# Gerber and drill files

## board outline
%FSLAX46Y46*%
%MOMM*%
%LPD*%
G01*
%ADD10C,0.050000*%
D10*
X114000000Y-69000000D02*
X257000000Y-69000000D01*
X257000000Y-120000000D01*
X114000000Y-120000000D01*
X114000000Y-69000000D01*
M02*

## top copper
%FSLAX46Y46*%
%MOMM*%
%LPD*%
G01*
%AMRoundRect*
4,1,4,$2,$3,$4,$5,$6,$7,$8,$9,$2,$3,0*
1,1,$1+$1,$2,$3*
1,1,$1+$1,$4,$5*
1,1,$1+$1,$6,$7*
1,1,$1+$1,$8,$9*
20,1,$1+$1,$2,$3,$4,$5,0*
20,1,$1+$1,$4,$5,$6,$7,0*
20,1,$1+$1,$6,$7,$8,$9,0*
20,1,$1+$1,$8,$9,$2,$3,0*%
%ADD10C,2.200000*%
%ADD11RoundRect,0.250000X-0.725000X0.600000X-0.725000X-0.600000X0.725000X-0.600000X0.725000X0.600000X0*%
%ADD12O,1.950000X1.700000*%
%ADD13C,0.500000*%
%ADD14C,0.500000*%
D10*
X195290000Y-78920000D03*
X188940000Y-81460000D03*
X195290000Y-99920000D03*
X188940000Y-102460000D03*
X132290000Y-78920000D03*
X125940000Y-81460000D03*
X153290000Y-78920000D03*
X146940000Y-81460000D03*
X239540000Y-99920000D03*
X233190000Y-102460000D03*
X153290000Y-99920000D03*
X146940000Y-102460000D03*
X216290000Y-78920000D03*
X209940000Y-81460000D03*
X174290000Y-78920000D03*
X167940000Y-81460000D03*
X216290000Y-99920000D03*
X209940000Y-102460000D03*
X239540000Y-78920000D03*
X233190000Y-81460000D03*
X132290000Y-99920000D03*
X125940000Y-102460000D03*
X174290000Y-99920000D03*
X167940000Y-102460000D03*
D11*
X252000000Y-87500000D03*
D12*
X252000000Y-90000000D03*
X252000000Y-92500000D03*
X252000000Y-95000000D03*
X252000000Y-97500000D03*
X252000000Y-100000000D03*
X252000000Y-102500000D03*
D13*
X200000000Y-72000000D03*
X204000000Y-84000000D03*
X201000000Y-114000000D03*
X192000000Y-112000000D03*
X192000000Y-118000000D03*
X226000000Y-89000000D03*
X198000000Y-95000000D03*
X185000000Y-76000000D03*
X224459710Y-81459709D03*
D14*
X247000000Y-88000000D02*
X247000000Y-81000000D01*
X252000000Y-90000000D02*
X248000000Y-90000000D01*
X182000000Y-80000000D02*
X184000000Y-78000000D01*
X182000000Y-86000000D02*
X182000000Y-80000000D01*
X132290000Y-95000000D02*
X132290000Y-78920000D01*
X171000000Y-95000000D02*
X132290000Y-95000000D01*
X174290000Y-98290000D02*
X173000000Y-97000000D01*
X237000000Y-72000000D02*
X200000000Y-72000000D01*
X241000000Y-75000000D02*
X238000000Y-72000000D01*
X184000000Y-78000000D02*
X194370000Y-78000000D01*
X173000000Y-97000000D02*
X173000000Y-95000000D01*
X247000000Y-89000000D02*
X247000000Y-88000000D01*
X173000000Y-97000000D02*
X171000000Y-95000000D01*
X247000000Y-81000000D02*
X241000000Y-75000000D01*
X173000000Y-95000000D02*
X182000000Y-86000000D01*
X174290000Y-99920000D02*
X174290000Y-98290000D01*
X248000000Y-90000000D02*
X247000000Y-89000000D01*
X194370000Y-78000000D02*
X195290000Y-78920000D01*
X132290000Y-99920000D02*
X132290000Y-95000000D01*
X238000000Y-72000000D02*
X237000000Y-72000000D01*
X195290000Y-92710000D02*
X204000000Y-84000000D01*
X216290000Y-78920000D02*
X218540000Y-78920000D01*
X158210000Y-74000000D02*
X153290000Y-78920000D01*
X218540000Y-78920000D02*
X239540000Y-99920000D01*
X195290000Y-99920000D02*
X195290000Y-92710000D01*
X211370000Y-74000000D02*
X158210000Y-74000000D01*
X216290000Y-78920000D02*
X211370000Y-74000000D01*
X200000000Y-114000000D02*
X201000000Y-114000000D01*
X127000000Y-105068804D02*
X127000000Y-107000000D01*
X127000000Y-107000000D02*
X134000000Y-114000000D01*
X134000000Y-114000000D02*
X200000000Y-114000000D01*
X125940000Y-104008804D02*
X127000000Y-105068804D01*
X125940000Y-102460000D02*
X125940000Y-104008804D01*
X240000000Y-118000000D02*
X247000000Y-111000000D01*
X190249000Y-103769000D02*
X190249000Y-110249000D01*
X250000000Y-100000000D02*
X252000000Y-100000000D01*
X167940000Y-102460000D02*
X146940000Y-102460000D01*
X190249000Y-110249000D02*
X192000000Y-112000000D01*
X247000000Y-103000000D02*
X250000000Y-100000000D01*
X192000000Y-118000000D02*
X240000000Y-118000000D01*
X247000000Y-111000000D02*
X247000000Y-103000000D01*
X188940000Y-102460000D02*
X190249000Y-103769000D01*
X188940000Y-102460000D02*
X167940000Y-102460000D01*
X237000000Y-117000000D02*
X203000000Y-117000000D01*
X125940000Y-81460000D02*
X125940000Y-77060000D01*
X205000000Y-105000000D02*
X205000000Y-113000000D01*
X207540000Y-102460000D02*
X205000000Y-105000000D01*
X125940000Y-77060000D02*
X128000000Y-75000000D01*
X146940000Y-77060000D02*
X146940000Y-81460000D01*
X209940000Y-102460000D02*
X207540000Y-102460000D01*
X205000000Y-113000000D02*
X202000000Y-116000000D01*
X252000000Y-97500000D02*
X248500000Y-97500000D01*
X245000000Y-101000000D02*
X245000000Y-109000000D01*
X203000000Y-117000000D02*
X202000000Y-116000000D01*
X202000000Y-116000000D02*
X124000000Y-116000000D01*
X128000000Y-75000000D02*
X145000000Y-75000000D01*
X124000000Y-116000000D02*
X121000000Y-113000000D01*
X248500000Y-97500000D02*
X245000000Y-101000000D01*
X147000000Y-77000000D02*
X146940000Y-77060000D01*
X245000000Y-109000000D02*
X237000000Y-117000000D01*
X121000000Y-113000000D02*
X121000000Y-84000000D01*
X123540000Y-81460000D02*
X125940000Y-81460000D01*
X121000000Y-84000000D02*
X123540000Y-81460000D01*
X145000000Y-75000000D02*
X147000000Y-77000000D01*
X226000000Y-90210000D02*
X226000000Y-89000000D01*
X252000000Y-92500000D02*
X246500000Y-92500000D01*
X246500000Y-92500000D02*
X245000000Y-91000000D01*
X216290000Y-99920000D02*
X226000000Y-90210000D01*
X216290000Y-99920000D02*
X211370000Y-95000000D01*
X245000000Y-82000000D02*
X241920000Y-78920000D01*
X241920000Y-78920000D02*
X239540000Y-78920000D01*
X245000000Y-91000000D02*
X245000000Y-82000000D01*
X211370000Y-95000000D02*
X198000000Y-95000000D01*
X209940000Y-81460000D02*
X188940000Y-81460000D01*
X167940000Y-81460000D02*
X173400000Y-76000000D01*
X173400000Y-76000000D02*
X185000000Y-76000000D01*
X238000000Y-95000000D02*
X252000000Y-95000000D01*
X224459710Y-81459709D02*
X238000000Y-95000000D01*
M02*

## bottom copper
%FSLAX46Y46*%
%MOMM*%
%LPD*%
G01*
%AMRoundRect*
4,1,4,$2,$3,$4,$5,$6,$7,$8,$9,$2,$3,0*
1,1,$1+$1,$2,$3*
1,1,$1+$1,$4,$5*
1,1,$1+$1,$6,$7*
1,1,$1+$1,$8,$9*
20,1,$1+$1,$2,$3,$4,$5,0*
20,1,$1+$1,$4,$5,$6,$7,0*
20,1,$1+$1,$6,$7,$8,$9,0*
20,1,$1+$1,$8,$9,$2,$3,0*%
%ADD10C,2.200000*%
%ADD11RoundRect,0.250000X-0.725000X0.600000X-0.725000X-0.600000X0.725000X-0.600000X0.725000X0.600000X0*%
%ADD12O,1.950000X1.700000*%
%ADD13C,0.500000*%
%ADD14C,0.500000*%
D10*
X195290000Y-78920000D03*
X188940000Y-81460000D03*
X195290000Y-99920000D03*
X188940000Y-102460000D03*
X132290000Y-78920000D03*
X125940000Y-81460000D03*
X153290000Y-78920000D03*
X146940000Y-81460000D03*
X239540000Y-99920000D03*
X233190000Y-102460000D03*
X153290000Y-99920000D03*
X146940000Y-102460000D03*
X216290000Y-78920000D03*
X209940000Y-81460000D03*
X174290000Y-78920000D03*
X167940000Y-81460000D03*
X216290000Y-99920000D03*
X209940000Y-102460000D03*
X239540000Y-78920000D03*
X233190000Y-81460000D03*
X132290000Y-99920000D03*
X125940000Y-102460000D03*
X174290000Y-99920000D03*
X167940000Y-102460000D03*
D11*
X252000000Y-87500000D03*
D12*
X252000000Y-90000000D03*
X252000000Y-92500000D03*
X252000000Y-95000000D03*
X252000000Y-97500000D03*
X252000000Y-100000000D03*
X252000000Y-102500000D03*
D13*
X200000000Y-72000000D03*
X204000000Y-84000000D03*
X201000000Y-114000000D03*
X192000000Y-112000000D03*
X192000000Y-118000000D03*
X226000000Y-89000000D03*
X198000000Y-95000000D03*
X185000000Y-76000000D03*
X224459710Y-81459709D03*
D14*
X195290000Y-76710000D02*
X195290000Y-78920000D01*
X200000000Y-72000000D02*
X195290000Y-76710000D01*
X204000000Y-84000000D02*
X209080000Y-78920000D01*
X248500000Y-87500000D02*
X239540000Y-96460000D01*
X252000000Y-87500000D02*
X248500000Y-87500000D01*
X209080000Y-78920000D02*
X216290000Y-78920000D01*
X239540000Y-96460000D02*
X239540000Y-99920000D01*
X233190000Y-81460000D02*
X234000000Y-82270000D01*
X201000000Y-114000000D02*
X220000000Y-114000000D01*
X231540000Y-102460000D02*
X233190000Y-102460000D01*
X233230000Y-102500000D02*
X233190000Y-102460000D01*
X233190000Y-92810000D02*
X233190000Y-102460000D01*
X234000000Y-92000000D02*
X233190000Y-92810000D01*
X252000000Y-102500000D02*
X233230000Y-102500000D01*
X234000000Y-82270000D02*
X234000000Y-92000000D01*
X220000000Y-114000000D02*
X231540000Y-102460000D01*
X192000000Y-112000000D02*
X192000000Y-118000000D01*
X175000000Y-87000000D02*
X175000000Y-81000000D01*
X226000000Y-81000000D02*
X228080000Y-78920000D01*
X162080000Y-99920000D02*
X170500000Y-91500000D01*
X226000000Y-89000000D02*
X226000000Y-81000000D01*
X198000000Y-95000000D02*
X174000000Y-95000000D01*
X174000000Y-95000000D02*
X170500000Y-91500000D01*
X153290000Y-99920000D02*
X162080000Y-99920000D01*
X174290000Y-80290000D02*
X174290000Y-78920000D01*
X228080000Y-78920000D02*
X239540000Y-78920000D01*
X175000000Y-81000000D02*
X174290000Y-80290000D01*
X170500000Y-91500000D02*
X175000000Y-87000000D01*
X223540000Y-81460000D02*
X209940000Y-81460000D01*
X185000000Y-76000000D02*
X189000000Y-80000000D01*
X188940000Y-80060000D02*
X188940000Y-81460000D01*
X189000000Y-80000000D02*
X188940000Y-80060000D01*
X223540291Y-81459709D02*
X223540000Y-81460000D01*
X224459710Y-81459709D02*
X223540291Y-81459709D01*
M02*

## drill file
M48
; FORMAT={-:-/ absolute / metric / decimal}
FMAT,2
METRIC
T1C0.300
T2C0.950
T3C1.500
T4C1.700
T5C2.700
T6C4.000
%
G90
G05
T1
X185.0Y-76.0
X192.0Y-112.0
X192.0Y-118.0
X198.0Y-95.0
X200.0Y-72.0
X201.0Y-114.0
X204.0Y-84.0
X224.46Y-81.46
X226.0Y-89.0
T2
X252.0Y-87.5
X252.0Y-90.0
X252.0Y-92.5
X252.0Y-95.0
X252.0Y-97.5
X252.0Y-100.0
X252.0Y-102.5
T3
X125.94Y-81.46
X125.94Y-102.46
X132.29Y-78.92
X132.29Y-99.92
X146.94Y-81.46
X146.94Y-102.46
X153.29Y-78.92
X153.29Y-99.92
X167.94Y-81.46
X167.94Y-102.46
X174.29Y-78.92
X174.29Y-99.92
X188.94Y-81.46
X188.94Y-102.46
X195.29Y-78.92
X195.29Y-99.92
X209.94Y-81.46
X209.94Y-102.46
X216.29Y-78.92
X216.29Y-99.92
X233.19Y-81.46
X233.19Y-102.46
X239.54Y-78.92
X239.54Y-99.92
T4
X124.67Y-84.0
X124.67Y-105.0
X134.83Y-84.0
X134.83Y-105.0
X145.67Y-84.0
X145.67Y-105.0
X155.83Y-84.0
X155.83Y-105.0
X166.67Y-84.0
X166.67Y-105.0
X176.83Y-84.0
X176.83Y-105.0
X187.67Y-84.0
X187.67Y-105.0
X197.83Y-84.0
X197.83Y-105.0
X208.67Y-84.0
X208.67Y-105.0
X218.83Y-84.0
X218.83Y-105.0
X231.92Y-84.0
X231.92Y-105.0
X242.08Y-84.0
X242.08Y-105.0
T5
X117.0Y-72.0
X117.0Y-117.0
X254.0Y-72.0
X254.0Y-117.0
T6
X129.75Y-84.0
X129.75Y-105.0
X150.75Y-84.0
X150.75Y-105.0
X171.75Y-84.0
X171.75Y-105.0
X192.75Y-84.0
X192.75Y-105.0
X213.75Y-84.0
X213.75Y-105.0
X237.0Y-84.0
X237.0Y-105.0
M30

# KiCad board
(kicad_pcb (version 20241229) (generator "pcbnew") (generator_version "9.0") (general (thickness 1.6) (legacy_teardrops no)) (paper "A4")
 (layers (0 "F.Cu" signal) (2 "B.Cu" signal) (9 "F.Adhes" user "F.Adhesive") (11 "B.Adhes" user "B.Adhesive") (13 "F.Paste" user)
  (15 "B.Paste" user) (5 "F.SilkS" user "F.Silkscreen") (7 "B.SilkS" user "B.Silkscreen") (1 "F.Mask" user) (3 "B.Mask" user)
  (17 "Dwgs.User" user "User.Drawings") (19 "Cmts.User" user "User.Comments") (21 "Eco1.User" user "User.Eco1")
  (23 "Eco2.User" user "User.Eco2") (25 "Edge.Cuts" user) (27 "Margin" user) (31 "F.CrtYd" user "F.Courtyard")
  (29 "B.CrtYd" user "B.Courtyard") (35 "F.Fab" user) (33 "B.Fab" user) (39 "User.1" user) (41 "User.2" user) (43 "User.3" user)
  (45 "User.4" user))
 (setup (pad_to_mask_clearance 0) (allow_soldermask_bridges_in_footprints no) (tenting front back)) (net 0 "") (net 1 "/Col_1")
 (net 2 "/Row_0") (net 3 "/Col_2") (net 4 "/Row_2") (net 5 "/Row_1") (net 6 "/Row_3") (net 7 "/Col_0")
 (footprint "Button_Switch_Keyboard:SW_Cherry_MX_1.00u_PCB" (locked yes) (layer "F.Cu") (at 195.29 78.92)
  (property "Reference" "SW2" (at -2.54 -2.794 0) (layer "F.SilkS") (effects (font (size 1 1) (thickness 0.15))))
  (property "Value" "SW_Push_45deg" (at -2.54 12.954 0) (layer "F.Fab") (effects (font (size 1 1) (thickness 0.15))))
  (pad "" np_thru_hole circle (at -7.62 5.08) (size 1.7 1.7) (drill 1.7) (layers "*.Cu" "*.Mask"))
  (pad "" np_thru_hole circle (at -2.54 5.08) (size 4 4) (drill 4) (layers "*.Cu" "*.Mask"))
  (pad "" np_thru_hole circle (at 2.54 5.08) (size 1.7 1.7) (drill 1.7) (layers "*.Cu" "*.Mask"))
  (pad "1" thru_hole circle (at 0 0) (size 2.2 2.2) (drill 1.5) (layers "*.Cu" "*.Mask") (remove_unused_layers no) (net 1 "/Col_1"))
  (pad "2" thru_hole circle (at -6.35 2.54) (size 2.2 2.2) (drill 1.5) (layers "*.Cu" "*.Mask") (remove_unused_layers no) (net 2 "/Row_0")))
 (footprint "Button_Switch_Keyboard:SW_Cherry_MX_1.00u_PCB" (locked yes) (layer "F.Cu") (at 195.29 99.92)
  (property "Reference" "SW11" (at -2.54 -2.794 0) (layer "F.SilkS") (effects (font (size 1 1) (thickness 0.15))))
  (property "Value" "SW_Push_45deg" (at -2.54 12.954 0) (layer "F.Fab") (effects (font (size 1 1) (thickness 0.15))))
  (pad "" np_thru_hole circle (at -7.62 5.08) (size 1.7 1.7) (drill 1.7) (layers "*.Cu" "*.Mask"))
  (pad "" np_thru_hole circle (at -2.54 5.08) (size 4 4) (drill 4) (layers "*.Cu" "*.Mask"))
  (pad "" np_thru_hole circle (at 2.54 5.08) (size 1.7 1.7) (drill 1.7) (layers "*.Cu" "*.Mask"))
  (pad "1" thru_hole circle (at 0 0) (size 2.2 2.2) (drill 1.5) (layers "*.Cu" "*.Mask") (remove_unused_layers no) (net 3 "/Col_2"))
  (pad "2" thru_hole circle (at -6.35 2.54) (size 2.2 2.2) (drill 1.5) (layers "*.Cu" "*.Mask") (remove_unused_layers no) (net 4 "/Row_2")))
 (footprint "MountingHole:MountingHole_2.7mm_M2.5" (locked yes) (layer "F.Cu") (at 117 72)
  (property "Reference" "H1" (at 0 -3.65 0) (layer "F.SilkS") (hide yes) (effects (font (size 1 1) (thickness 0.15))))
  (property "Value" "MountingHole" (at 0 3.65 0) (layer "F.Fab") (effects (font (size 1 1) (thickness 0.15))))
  (pad "" np_thru_hole circle (at 0 0) (size 2.7 2.7) (drill 2.7) (layers "*.Cu" "*.Mask")))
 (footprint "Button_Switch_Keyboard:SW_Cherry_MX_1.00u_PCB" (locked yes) (layer "F.Cu") (at 132.29 78.92)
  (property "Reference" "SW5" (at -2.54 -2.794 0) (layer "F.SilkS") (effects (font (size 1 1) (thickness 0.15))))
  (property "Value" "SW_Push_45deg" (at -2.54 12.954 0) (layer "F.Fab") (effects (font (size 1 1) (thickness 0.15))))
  (pad "" np_thru_hole circle (at -7.62 5.08) (size 1.7 1.7) (drill 1.7) (layers "*.Cu" "*.Mask"))
  (pad "" np_thru_hole circle (at -2.54 5.08) (size 4 4) (drill 4) (layers "*.Cu" "*.Mask"))
  (pad "" np_thru_hole circle (at 2.54 5.08) (size 1.7 1.7) (drill 1.7) (layers "*.Cu" "*.Mask"))
  (pad "1" thru_hole circle (at 0 0) (size 2.2 2.2) (drill 1.5) (layers "*.Cu" "*.Mask") (remove_unused_layers no) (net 1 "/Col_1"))
  (pad "2" thru_hole circle (at -6.35 2.54) (size 2.2 2.2) (drill 1.5) (layers "*.Cu" "*.Mask") (remove_unused_layers no) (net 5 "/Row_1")))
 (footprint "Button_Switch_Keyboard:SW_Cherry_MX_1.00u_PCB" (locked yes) (layer "F.Cu") (at 153.29 78.92)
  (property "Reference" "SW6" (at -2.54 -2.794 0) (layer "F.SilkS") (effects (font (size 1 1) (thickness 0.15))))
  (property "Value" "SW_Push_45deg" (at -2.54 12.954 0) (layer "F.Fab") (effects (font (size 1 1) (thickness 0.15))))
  (pad "" np_thru_hole circle (at -7.62 5.08) (size 1.7 1.7) (drill 1.7) (layers "*.Cu" "*.Mask"))
  (pad "" np_thru_hole circle (at -2.54 5.08) (size 4 4) (drill 4) (layers "*.Cu" "*.Mask"))
  (pad "" np_thru_hole circle (at 2.54 5.08) (size 1.7 1.7) (drill 1.7) (layers "*.Cu" "*.Mask"))
  (pad "1" thru_hole circle (at 0 0) (size 2.2 2.2) (drill 1.5) (layers "*.Cu" "*.Mask") (remove_unused_layers no) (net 3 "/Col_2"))
  (pad "2" thru_hole circle (at -6.35 2.54) (size 2.2 2.2) (drill 1.5) (layers "*.Cu" "*.Mask") (remove_unused_layers no) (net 5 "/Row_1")))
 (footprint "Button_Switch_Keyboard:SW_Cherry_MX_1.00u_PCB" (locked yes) (layer "F.Cu") (at 239.54 99.92)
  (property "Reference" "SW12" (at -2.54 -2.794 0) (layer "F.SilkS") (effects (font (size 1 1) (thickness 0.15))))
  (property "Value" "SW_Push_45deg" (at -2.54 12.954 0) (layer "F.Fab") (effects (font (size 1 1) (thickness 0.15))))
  (pad "" np_thru_hole circle (at -7.62 5.08) (size 1.7 1.7) (drill 1.7) (layers "*.Cu" "*.Mask"))
  (pad "" np_thru_hole circle (at -2.54 5.08) (size 4 4) (drill 4) (layers "*.Cu" "*.Mask"))
  (pad "" np_thru_hole circle (at 2.54 5.08) (size 1.7 1.7) (drill 1.7) (layers "*.Cu" "*.Mask"))
  (pad "1" thru_hole circle (at 0 0) (size 2.2 2.2) (drill 1.5) (layers "*.Cu" "*.Mask") (remove_unused_layers no) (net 3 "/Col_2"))
  (pad "2" thru_hole circle (at -6.35 2.54) (size 2.2 2.2) (drill 1.5) (layers "*.Cu" "*.Mask") (remove_unused_layers no) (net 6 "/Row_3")))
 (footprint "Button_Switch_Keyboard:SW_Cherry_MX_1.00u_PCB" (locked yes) (layer "F.Cu") (at 153.29 99.92)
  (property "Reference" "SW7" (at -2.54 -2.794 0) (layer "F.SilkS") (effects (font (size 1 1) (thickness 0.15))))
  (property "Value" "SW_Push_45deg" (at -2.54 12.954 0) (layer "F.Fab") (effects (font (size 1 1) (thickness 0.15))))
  (pad "" np_thru_hole circle (at -7.62 5.08) (size 1.7 1.7) (drill 1.7) (layers "*.Cu" "*.Mask"))
  (pad "" np_thru_hole circle (at -2.54 5.08) (size 4 4) (drill 4) (layers "*.Cu" "*.Mask"))
  (pad "" np_thru_hole circle (at 2.54 5.08) (size 1.7 1.7) (drill 1.7) (layers "*.Cu" "*.Mask"))
  (pad "1" thru_hole circle (at 0 0) (size 2.2 2.2) (drill 1.5) (layers "*.Cu" "*.Mask") (remove_unused_layers no) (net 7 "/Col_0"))
  (pad "2" thru_hole circle (at -6.35 2.54) (size 2.2 2.2) (drill 1.5) (layers "*.Cu" "*.Mask") (remove_unused_layers no) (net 4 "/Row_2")))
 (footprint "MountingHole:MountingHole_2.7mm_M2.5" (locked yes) (layer "F.Cu") (at 254 117)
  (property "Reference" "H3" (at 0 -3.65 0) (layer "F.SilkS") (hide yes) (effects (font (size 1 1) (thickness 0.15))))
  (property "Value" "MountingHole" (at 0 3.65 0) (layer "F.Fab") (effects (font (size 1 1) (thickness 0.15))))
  (pad "" np_thru_hole circle (at 0 0) (size 2.7 2.7) (drill 2.7) (layers "*.Cu" "*.Mask")))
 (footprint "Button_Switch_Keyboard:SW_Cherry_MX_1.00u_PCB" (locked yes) (layer "F.Cu") (at 216.29 78.92)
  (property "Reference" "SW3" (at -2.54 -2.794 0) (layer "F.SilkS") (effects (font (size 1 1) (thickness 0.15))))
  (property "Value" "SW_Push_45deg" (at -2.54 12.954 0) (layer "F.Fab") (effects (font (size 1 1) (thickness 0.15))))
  (pad "" np_thru_hole circle (at -7.62 5.08) (size 1.7 1.7) (drill 1.7) (layers "*.Cu" "*.Mask"))
  (pad "" np_thru_hole circle (at -2.54 5.08) (size 4 4) (drill 4) (layers "*.Cu" "*.Mask"))
  (pad "" np_thru_hole circle (at 2.54 5.08) (size 1.7 1.7) (drill 1.7) (layers "*.Cu" "*.Mask"))
  (pad "1" thru_hole circle (at 0 0) (size 2.2 2.2) (drill 1.5) (layers "*.Cu" "*.Mask") (remove_unused_layers no) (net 3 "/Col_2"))
  (pad "2" thru_hole circle (at -6.35 2.54) (size 2.2 2.2) (drill 1.5) (layers "*.Cu" "*.Mask") (remove_unused_layers no) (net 2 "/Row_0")))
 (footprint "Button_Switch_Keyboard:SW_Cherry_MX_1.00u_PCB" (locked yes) (layer "F.Cu") (at 174.29 78.92)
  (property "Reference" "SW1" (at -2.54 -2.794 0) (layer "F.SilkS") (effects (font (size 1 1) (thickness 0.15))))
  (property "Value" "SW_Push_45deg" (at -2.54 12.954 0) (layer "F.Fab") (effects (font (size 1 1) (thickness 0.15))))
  (pad "" np_thru_hole circle (at -7.62 5.08) (size 1.7 1.7) (drill 1.7) (layers "*.Cu" "*.Mask"))
  (pad "" np_thru_hole circle (at -2.54 5.08) (size 4 4) (drill 4) (layers "*.Cu" "*.Mask"))
  (pad "" np_thru_hole circle (at 2.54 5.08) (size 1.7 1.7) (drill 1.7) (layers "*.Cu" "*.Mask"))
  (pad "1" thru_hole circle (at 0 0) (size 2.2 2.2) (drill 1.5) (layers "*.Cu" "*.Mask") (remove_unused_layers no) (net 7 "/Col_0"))
  (pad "2" thru_hole circle (at -6.35 2.54) (size 2.2 2.2) (drill 1.5) (layers "*.Cu" "*.Mask") (remove_unused_layers no) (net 2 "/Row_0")))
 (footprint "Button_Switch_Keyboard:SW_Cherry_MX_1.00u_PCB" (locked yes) (layer "F.Cu") (at 216.29 99.92)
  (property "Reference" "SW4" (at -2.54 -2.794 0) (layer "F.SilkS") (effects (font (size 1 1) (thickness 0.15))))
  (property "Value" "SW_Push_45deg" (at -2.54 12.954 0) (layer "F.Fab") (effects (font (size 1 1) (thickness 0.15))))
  (pad "" np_thru_hole circle (at -7.62 5.08) (size 1.7 1.7) (drill 1.7) (layers "*.Cu" "*.Mask"))
  (pad "" np_thru_hole circle (at -2.54 5.08) (size 4 4) (drill 4) (layers "*.Cu" "*.Mask"))
  (pad "" np_thru_hole circle (at 2.54 5.08) (size 1.7 1.7) (drill 1.7) (layers "*.Cu" "*.Mask"))
  (pad "1" thru_hole circle (at 0 0) (size 2.2 2.2) (drill 1.5) (layers "*.Cu" "*.Mask") (remove_unused_layers no) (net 7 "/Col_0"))
  (pad "2" thru_hole circle (at -6.35 2.54) (size 2.2 2.2) (drill 1.5) (layers "*.Cu" "*.Mask") (remove_unused_layers no) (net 5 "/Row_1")))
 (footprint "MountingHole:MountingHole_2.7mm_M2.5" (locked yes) (layer "F.Cu") (at 117 117)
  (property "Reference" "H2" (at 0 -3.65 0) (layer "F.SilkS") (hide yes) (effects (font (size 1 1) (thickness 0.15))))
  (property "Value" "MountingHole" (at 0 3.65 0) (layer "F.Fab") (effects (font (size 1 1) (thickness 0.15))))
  (pad "" np_thru_hole circle (at 0 0) (size 2.7 2.7) (drill 2.7) (layers "*.Cu" "*.Mask")))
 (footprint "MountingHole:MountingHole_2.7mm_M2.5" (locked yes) (layer "F.Cu") (at 254 72)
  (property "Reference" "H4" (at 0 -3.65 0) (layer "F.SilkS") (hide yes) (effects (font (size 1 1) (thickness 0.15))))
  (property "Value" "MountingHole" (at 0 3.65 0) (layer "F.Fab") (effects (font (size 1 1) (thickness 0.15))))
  (pad "" np_thru_hole circle (at 0 0) (size 2.7 2.7) (drill 2.7) (layers "*.Cu" "*.Mask")))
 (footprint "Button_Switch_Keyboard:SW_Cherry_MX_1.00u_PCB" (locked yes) (layer "F.Cu") (at 239.54 78.92)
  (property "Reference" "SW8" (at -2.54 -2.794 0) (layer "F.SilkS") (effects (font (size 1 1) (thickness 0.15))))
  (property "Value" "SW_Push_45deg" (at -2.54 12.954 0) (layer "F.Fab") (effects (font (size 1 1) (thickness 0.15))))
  (pad "" np_thru_hole circle (at -7.62 5.08) (size 1.7 1.7) (drill 1.7) (layers "*.Cu" "*.Mask"))
  (pad "" np_thru_hole circle (at -2.54 5.08) (size 4 4) (drill 4) (layers "*.Cu" "*.Mask"))
  (pad "" np_thru_hole circle (at 2.54 5.08) (size 1.7 1.7) (drill 1.7) (layers "*.Cu" "*.Mask"))
  (pad "1" thru_hole circle (at 0 0) (size 2.2 2.2) (drill 1.5) (layers "*.Cu" "*.Mask") (remove_unused_layers no) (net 7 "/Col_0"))
  (pad "2" thru_hole circle (at -6.35 2.54) (size 2.2 2.2) (drill 1.5) (layers "*.Cu" "*.Mask") (remove_unused_layers no) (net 6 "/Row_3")))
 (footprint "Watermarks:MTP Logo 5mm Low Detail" (layer "F.Cu") (at 226 117)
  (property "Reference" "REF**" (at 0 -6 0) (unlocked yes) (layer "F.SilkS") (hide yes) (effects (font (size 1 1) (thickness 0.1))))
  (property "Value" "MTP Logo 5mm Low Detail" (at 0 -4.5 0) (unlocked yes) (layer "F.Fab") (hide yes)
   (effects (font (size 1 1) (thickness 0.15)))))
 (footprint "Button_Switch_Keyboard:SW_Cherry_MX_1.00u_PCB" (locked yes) (layer "F.Cu") (at 132.29 99.92)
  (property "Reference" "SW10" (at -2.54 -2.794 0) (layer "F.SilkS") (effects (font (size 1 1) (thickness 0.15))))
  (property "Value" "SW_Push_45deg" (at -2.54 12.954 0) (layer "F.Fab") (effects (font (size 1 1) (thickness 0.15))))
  (pad "" np_thru_hole circle (at -7.62 5.08) (size 1.7 1.7) (drill 1.7) (layers "*.Cu" "*.Mask"))
  (pad "" np_thru_hole circle (at -2.54 5.08) (size 4 4) (drill 4) (layers "*.Cu" "*.Mask"))
  (pad "" np_thru_hole circle (at 2.54 5.08) (size 1.7 1.7) (drill 1.7) (layers "*.Cu" "*.Mask"))
  (pad "1" thru_hole circle (at 0 0) (size 2.2 2.2) (drill 1.5) (layers "*.Cu" "*.Mask") (remove_unused_layers no) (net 1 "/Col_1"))
  (pad "2" thru_hole circle (at -6.35 2.54) (size 2.2 2.2) (drill 1.5) (layers "*.Cu" "*.Mask") (remove_unused_layers no) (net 6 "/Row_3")))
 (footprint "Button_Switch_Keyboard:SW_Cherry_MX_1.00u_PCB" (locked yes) (layer "F.Cu") (at 174.29 99.92)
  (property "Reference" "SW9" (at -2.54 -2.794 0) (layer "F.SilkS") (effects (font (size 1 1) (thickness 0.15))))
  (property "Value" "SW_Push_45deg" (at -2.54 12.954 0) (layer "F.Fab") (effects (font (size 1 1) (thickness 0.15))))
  (pad "" np_thru_hole circle (at -7.62 5.08) (size 1.7 1.7) (drill 1.7) (layers "*.Cu" "*.Mask"))
  (pad "" np_thru_hole circle (at -2.54 5.08) (size 4 4) (drill 4) (layers "*.Cu" "*.Mask"))
  (pad "" np_thru_hole circle (at 2.54 5.08) (size 1.7 1.7) (drill 1.7) (layers "*.Cu" "*.Mask"))
  (pad "1" thru_hole circle (at 0 0) (size 2.2 2.2) (drill 1.5) (layers "*.Cu" "*.Mask") (remove_unused_layers no) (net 1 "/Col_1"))
  (pad "2" thru_hole circle (at -6.35 2.54) (size 2.2 2.2) (drill 1.5) (layers "*.Cu" "*.Mask") (remove_unused_layers no) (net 4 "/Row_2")))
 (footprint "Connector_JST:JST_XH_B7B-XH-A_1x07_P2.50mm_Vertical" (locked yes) (layer "B.Cu") (at 252 87.5 -90)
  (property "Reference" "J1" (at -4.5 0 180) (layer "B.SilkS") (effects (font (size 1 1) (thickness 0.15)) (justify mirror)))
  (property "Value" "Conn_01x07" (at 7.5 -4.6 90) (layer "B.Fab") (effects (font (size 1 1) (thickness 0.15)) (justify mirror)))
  (pad "1" thru_hole roundrect (at 0 0 270) (size 1.7 1.95) (drill 0.95) (layers "*.Cu" "*.Mask") (remove_unused_layers no)
   (roundrect_rratio 0.147059) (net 3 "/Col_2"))
  (pad "2" thru_hole oval (at 2.5 0 270) (size 1.7 1.95) (drill 0.95) (layers "*.Cu" "*.Mask") (remove_unused_layers no) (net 1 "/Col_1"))
  (pad "3" thru_hole oval (at 5 0 270) (size 1.7 1.95) (drill 0.95) (layers "*.Cu" "*.Mask") (remove_unused_layers no) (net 7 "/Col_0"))
  (pad "4" thru_hole oval (at 7.5 0 270) (size 1.7 1.95) (drill 0.95) (layers "*.Cu" "*.Mask") (remove_unused_layers no) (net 2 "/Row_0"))
  (pad "5" thru_hole oval (at 10 0 270) (size 1.7 1.95) (drill 0.95) (layers "*.Cu" "*.Mask") (remove_unused_layers no) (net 5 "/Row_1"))
  (pad "6" thru_hole oval (at 12.5 0 270) (size 1.7 1.95) (drill 0.95) (layers "*.Cu" "*.Mask") (remove_unused_layers no) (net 4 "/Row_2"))
  (pad "7" thru_hole oval (at 15 0 270) (size 1.7 1.95) (drill 0.95) (layers "*.Cu" "*.Mask") (remove_unused_layers no) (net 6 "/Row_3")))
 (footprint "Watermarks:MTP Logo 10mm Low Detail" (layer "B.Cu") (at 187.465327 92.158133 180)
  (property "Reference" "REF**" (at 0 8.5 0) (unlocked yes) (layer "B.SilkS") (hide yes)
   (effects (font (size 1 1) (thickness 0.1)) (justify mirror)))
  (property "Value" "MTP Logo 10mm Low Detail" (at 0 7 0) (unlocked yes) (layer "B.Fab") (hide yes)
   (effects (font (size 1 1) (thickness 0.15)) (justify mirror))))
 (gr_rect (start 114 69) (end 257 120) (stroke (width 0.05) (type solid)) (fill no) (locked yes) (layer "Edge.Cuts"))
 (segment (start 247 88) (end 247 81) (width 0.5) (layer "F.Cu") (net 1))
 (segment (start 252 90) (end 248 90) (width 0.5) (layer "F.Cu") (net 1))
 (segment (start 182 80) (end 184 78) (width 0.5) (layer "F.Cu") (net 1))
 (segment (start 182 86) (end 182 80) (width 0.5) (layer "F.Cu") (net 1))
 (segment (start 132.29 95) (end 132.29 78.92) (width 0.5) (layer "F.Cu") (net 1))
 (segment (start 171 95) (end 132.29 95) (width 0.5) (layer "F.Cu") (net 1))
 (segment (start 174.29 98.29) (end 173 97) (width 0.5) (layer "F.Cu") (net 1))
 (segment (start 237 72) (end 200 72) (width 0.5) (layer "F.Cu") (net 1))
 (segment (start 241 75) (end 238 72) (width 0.5) (layer "F.Cu") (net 1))
 (segment (start 184 78) (end 194.37 78) (width 0.5) (layer "F.Cu") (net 1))
 (segment (start 173 97) (end 173 95) (width 0.5) (layer "F.Cu") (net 1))
 (segment (start 247 89) (end 247 88) (width 0.5) (layer "F.Cu") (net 1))
 (segment (start 173 97) (end 171 95) (width 0.5) (layer "F.Cu") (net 1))
 (segment (start 247 81) (end 241 75) (width 0.5) (layer "F.Cu") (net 1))
 (segment (start 173 95) (end 182 86) (width 0.5) (layer "F.Cu") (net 1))
 (segment (start 174.29 99.92) (end 174.29 98.29) (width 0.5) (layer "F.Cu") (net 1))
 (segment (start 248 90) (end 247 89) (width 0.5) (layer "F.Cu") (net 1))
 (segment (start 194.37 78) (end 195.29 78.92) (width 0.5) (layer "F.Cu") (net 1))
 (segment (start 132.29 99.92) (end 132.29 95) (width 0.5) (layer "F.Cu") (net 1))
 (segment (start 238 72) (end 237 72) (width 0.5) (layer "F.Cu") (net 1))
 (via (at 200 72) (size 0.5) (drill 0.3) (layers "F.Cu" "B.Cu") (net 1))
 (segment (start 195.29 76.71) (end 195.29 78.92) (width 0.5) (layer "B.Cu") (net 1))
 (segment (start 200 72) (end 195.29 76.71) (width 0.5) (layer "B.Cu") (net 1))
 (segment (start 195.29 92.71) (end 204 84) (width 0.5) (layer "F.Cu") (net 3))
 (segment (start 216.29 78.92) (end 218.54 78.92) (width 0.5) (layer "F.Cu") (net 3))
 (segment (start 158.21 74) (end 153.29 78.92) (width 0.5) (layer "F.Cu") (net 3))
 (segment (start 218.54 78.92) (end 239.54 99.92) (width 0.5) (layer "F.Cu") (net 3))
 (segment (start 195.29 99.92) (end 195.29 92.71) (width 0.5) (layer "F.Cu") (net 3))
 (segment (start 211.37 74) (end 158.21 74) (width 0.5) (layer "F.Cu") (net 3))
 (segment (start 216.29 78.92) (end 211.37 74) (width 0.5) (layer "F.Cu") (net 3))
 (via (at 204 84) (size 0.5) (drill 0.3) (layers "F.Cu" "B.Cu") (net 3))
 (segment (start 204 84) (end 209.08 78.92) (width 0.5) (layer "B.Cu") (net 3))
 (segment (start 248.5 87.5) (end 239.54 96.46) (width 0.5) (layer "B.Cu") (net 3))
 (segment (start 252 87.5) (end 248.5 87.5) (width 0.5) (layer "B.Cu") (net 3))
 (segment (start 209.08 78.92) (end 216.29 78.92) (width 0.5) (layer "B.Cu") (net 3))
 (segment (start 239.54 96.46) (end 239.54 99.92) (width 0.5) (layer "B.Cu") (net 3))
 (segment (start 200 114) (end 201 114) (width 0.5) (layer "F.Cu") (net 6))
 (segment (start 127 105.068804) (end 127 107) (width 0.5) (layer "F.Cu") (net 6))
 (segment (start 127 107) (end 134 114) (width 0.5) (layer "F.Cu") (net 6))
 (segment (start 134 114) (end 200 114) (width 0.5) (layer "F.Cu") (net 6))
 (segment (start 125.94 104.008804) (end 127 105.068804) (width 0.5) (layer "F.Cu") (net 6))
 (segment (start 125.94 102.46) (end 125.94 104.008804) (width 0.5) (layer "F.Cu") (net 6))
 (via (at 201 114) (size 0.5) (drill 0.3) (layers "F.Cu" "B.Cu") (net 6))
 (segment (start 233.19 81.46) (end 234 82.27) (width 0.5) (layer "B.Cu") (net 6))
 (segment (start 201 114) (end 220 114) (width 0.5) (layer "B.Cu") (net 6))
 (segment (start 231.54 102.46) (end 233.19 102.46) (width 0.5) (layer "B.Cu") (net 6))
 (segment (start 233.23 102.5) (end 233.19 102.46) (width 0.5) (layer "B.Cu") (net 6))
 (segment (start 233.19 92.81) (end 233.19 102.46) (width 0.5) (layer "B.Cu") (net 6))
 (segment (start 234 92) (end 233.19 92.81) (width 0.5) (layer "B.Cu") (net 6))
 (segment (start 252 102.5) (end 233.23 102.5) (width 0.5) (layer "B.Cu") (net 6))
 (segment (start 234 82.27) (end 234 92) (width 0.5) (layer "B.Cu") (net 6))
 (segment (start 220 114) (end 231.54 102.46) (width 0.5) (layer "B.Cu") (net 6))
 (segment (start 240 118) (end 247 111) (width 0.5) (layer "F.Cu") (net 4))
 (segment (start 190.249 103.769) (end 190.249 110.249) (width 0.5) (layer "F.Cu") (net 4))
 (segment (start 250 100) (end 252 100) (width 0.5) (layer "F.Cu") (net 4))
 (segment (start 167.94 102.46) (end 146.94 102.46) (width 0.5) (layer "F.Cu") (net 4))
 (segment (start 190.249 110.249) (end 192 112) (width 0.5) (layer "F.Cu") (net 4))
 (segment (start 247 103) (end 250 100) (width 0.5) (layer "F.Cu") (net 4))
 (segment (start 192 118) (end 240 118) (width 0.5) (layer "F.Cu") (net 4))
 (segment (start 247 111) (end 247 103) (width 0.5) (layer "F.Cu") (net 4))
 (segment (start 188.94 102.46) (end 190.249 103.769) (width 0.5) (layer "F.Cu") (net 4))
 (segment (start 188.94 102.46) (end 167.94 102.46) (width 0.5) (layer "F.Cu") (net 4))
 (via (at 192 112) (size 0.5) (drill 0.3) (layers "F.Cu" "B.Cu") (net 4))
 (via (at 192 118) (size 0.5) (drill 0.3) (layers "F.Cu" "B.Cu") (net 4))
 (segment (start 192 112) (end 192 118) (width 0.5) (layer "B.Cu") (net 4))
 (segment (start 237 117) (end 203 117) (width 0.5) (layer "F.Cu") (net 5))
 (segment (start 125.94 81.46) (end 125.94 77.06) (width 0.5) (layer "F.Cu") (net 5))
 (segment (start 205 105) (end 205 113) (width 0.5) (layer "F.Cu") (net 5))
 (segment (start 207.54 102.46) (end 205 105) (width 0.5) (layer "F.Cu") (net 5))
 (segment (start 125.94 77.06) (end 128 75) (width 0.5) (layer "F.Cu") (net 5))
 (segment (start 146.94 77.06) (end 146.94 81.46) (width 0.5) (layer "F.Cu") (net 5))
 (segment (start 209.94 102.46) (end 207.54 102.46) (width 0.5) (layer "F.Cu") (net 5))
 (segment (start 205 113) (end 202 116) (width 0.5) (layer "F.Cu") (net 5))
 (segment (start 252 97.5) (end 248.5 97.5) (width 0.5) (layer "F.Cu") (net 5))
 (segment (start 245 101) (end 245 109) (width 0.5) (layer "F.Cu") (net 5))
 (segment (start 203 117) (end 202 116) (width 0.5) (layer "F.Cu") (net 5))
 (segment (start 202 116) (end 124 116) (width 0.5) (layer "F.Cu") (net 5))
 (segment (start 128 75) (end 145 75) (width 0.5) (layer "F.Cu") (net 5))
 (segment (start 124 116) (end 121 113) (width 0.5) (layer "F.Cu") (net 5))
 (segment (start 248.5 97.5) (end 245 101) (width 0.5) (layer "F.Cu") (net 5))
 (segment (start 147 77) (end 146.94 77.06) (width 0.5) (layer "F.Cu") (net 5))
 (segment (start 245 109) (end 237 117) (width 0.5) (layer "F.Cu") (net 5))
 (segment (start 121 113) (end 121 84) (width 0.5) (layer "F.Cu") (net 5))
 (segment (start 123.54 81.46) (end 125.94 81.46) (width 0.5) (layer "F.Cu") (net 5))
 (segment (start 121 84) (end 123.54 81.46) (width 0.5) (layer "F.Cu") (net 5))
 (segment (start 145 75) (end 147 77) (width 0.5) (layer "F.Cu") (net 5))
 (segment (start 226 90.21) (end 226 89) (width 0.5) (layer "F.Cu") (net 7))
 (segment (start 252 92.5) (end 246.5 92.5) (width 0.5) (layer "F.Cu") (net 7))
 (segment (start 246.5 92.5) (end 245 91) (width 0.5) (layer "F.Cu") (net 7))
 (segment (start 216.29 99.92) (end 226 90.21) (width 0.5) (layer "F.Cu") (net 7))
 (segment (start 216.29 99.92) (end 211.37 95) (width 0.5) (layer "F.Cu") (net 7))
 (segment (start 245 82) (end 241.92 78.92) (width 0.5) (layer "F.Cu") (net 7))
 (segment (start 241.92 78.92) (end 239.54 78.92) (width 0.5) (layer "F.Cu") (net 7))
 (segment (start 245 91) (end 245 82) (width 0.5) (layer "F.Cu") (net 7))
 (segment (start 211.37 95) (end 198 95) (width 0.5) (layer "F.Cu") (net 7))
 (via (at 226 89) (size 0.5) (drill 0.3) (layers "F.Cu" "B.Cu") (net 7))
 (via (at 198 95) (size 0.5) (drill 0.3) (layers "F.Cu" "B.Cu") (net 7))
 (segment (start 175 87) (end 175 81) (width 0.5) (layer "B.Cu") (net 7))
 (segment (start 226 81) (end 228.08 78.92) (width 0.5) (layer "B.Cu") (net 7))
 (segment (start 162.08 99.92) (end 170.5 91.5) (width 0.5) (layer "B.Cu") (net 7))
 (segment (start 226 89) (end 226 81) (width 0.5) (layer "B.Cu") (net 7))
 (segment (start 198 95) (end 174 95) (width 0.5) (layer "B.Cu") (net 7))
 (segment (start 174 95) (end 170.5 91.5) (width 0.5) (layer "B.Cu") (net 7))
 (segment (start 153.29 99.92) (end 162.08 99.92) (width 0.5) (layer "B.Cu") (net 7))
 (segment (start 174.29 80.29) (end 174.29 78.92) (width 0.5) (layer "B.Cu") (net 7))
 (segment (start 228.08 78.92) (end 239.54 78.92) (width 0.5) (layer "B.Cu") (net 7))
 (segment (start 175 81) (end 174.29 80.29) (width 0.5) (layer "B.Cu") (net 7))
 (segment (start 170.5 91.5) (end 175 87) (width 0.5) (layer "B.Cu") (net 7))
 (segment (start 209.94 81.46) (end 188.94 81.46) (width 0.5) (layer "F.Cu") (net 2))
 (segment (start 167.94 81.46) (end 173.4 76) (width 0.5) (layer "F.Cu") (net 2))
 (segment (start 173.4 76) (end 185 76) (width 0.5) (layer "F.Cu") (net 2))
 (segment (start 238 95) (end 252 95) (width 0.5) (layer "F.Cu") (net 2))
 (segment (start 224.45971 81.459709) (end 238 95) (width 0.5) (layer "F.Cu") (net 2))
 (via (at 185 76) (size 0.5) (drill 0.3) (layers "F.Cu" "B.Cu") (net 2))
 (via (at 224.45971 81.459709) (size 0.5) (drill 0.3) (layers "F.Cu" "B.Cu") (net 2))
 (segment (start 223.54 81.46) (end 209.94 81.46) (width 0.5) (layer "B.Cu") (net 2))
 (segment (start 185 76) (end 189 80) (width 0.5) (layer "B.Cu") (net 2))
 (segment (start 188.94 80.06) (end 188.94 81.46) (width 0.5) (layer "B.Cu") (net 2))
 (segment (start 189 80) (end 188.94 80.06) (width 0.5) (layer "B.Cu") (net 2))
 (segment (start 223.540291 81.459709) (end 223.54 81.46) (width 0.5) (layer "B.Cu") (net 2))
 (segment (start 224.45971 81.459709) (end 223.540291 81.459709) (width 0.5) (layer "B.Cu") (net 2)))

